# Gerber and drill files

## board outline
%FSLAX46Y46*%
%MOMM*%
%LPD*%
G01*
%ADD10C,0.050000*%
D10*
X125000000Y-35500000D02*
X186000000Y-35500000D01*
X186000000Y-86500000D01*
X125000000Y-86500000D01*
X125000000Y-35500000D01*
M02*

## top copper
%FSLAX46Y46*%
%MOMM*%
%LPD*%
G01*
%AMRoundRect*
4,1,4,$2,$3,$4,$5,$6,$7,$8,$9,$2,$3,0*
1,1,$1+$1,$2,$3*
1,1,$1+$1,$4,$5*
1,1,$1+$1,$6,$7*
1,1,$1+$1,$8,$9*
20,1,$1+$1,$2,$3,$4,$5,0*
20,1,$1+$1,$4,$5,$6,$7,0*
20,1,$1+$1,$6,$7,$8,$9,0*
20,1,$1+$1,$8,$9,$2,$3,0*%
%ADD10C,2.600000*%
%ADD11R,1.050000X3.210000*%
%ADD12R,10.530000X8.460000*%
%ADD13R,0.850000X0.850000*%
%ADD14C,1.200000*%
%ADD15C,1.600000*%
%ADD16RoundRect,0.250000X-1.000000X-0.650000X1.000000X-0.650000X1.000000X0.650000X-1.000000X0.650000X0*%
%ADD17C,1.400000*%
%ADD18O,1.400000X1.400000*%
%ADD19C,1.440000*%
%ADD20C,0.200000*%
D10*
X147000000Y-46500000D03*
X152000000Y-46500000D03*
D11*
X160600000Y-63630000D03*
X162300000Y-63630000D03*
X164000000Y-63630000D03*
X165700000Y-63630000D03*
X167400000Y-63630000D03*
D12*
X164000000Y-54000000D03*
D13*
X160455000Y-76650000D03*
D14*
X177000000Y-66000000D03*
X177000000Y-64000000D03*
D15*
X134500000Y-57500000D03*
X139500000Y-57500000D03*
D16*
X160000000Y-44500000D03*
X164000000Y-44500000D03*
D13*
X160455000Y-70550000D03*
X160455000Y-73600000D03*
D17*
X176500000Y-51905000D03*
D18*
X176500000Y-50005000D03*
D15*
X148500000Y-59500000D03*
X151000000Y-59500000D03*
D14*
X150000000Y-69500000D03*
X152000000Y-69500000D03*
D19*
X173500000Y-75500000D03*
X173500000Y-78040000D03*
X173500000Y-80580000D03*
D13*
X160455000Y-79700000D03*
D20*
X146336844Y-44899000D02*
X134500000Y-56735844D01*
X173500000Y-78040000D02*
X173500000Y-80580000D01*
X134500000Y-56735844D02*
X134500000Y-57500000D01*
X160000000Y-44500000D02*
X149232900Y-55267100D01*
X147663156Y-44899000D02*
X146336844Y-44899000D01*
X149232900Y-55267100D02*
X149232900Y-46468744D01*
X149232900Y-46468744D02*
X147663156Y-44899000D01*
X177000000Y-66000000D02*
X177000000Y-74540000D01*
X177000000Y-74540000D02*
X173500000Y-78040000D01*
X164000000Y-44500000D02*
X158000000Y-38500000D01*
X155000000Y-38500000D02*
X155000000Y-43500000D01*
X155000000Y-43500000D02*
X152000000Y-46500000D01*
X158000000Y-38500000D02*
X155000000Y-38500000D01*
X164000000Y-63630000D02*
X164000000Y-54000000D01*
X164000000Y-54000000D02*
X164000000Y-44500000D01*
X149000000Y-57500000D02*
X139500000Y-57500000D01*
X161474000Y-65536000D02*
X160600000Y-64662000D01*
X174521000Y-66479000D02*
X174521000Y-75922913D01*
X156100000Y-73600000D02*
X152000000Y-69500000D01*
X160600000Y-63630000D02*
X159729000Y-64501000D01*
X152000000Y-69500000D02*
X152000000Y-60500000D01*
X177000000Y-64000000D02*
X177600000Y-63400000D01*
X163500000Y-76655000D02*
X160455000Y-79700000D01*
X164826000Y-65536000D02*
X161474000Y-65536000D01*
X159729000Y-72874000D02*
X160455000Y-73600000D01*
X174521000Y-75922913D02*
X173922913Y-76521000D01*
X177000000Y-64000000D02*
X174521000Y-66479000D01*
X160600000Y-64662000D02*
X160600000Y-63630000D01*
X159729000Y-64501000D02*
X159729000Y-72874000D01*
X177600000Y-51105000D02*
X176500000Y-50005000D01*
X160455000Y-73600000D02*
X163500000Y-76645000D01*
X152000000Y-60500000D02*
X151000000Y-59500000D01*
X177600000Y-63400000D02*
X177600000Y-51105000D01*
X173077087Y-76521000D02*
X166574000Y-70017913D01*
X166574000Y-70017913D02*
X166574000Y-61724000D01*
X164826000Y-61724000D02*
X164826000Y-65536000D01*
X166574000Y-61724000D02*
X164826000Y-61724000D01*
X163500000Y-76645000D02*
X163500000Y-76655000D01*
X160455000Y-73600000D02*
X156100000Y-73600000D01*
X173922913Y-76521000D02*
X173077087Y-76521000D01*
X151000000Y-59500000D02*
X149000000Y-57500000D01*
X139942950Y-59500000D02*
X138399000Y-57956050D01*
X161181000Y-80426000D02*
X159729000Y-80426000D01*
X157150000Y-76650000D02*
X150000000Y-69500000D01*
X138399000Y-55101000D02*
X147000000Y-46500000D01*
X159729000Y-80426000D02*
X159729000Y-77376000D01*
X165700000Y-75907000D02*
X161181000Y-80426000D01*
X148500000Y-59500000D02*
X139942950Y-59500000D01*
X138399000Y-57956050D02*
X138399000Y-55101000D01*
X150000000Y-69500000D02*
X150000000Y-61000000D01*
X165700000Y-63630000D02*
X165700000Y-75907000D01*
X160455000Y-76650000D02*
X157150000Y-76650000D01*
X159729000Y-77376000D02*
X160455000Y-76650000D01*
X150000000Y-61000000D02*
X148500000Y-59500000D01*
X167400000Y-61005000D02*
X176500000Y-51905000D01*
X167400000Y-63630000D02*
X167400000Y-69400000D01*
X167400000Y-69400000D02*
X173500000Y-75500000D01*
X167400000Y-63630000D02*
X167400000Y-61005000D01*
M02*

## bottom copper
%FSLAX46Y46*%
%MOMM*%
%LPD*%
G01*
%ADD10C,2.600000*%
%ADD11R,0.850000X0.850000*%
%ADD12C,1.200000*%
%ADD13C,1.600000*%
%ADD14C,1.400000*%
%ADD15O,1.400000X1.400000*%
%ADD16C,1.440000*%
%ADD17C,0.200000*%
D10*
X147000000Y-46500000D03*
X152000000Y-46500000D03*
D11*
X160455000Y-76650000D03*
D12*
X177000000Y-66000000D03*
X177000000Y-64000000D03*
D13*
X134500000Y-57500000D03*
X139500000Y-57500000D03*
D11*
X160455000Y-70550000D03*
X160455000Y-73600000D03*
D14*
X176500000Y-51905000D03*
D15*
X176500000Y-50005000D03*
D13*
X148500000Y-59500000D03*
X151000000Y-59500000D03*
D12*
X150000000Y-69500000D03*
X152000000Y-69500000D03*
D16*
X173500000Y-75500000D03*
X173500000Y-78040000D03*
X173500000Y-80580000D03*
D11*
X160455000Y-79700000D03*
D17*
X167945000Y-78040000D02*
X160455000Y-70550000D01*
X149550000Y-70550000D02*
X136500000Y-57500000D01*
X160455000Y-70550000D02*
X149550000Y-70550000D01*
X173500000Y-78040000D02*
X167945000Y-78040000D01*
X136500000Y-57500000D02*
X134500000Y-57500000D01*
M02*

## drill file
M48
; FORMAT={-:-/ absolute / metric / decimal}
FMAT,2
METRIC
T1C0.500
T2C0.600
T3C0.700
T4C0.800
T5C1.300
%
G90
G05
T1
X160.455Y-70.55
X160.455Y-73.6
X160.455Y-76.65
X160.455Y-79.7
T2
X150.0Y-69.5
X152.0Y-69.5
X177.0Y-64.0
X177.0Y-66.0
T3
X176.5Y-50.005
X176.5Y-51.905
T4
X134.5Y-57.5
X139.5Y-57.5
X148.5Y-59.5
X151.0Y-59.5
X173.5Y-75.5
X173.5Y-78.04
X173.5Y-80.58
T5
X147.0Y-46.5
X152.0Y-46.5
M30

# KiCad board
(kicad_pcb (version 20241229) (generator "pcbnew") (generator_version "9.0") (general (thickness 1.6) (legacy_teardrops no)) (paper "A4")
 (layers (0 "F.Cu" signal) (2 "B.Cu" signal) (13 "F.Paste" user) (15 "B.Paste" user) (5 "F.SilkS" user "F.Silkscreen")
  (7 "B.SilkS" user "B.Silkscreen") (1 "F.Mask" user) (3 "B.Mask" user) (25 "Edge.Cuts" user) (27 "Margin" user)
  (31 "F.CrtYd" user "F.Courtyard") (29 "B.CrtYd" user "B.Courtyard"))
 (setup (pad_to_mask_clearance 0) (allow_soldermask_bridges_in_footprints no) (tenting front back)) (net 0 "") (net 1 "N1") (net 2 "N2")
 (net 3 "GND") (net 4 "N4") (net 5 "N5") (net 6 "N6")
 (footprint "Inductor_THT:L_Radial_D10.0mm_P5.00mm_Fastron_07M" (layer "F.Cu") (at 147 46.5)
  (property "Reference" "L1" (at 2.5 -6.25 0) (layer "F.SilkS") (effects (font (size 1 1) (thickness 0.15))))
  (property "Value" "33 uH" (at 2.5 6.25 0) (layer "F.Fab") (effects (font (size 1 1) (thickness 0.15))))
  (pad "1" thru_hole circle (at 0 0) (size 2.6 2.6) (drill 1.3) (layers "*.Cu" "*.Mask") (remove_unused_layers no) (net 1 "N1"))
  (pad "2" thru_hole circle (at 5 0) (size 2.6 2.6) (drill 1.3) (layers "*.Cu" "*.Mask") (remove_unused_layers no) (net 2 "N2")))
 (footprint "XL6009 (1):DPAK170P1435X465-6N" (layer "F.Cu") (at 164 57.5 90)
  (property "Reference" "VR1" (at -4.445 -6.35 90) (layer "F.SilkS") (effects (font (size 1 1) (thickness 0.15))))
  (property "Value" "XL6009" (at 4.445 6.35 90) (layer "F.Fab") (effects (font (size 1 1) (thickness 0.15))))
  (pad "1" smd rect (at -6.13 -3.4 90) (size 3.21 1.05) (layers "F.Cu" "F.Mask" "F.Paste") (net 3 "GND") (solder_mask_margin 0.102))
  (pad "2" smd rect (at -6.13 -1.7 90) (size 3.21 1.05) (layers "F.Cu" "F.Mask" "F.Paste") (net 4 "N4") (solder_mask_margin 0.102))
  (pad "3" smd rect (at -6.13 0 90) (size 3.21 1.05) (layers "F.Cu" "F.Mask" "F.Paste") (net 2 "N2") (solder_mask_margin 0.102))
  (pad "4" smd rect (at -6.13 1.7 90) (size 3.21 1.05) (layers "F.Cu" "F.Mask" "F.Paste") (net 1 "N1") (solder_mask_margin 0.102))
  (pad "5" smd rect (at -6.13 3.4 90) (size 3.21 1.05) (layers "F.Cu" "F.Mask" "F.Paste") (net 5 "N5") (solder_mask_margin 0.102))
  (pad "6" smd rect (at 3.5 0 90) (size 8.46 10.53) (layers "F.Cu" "F.Mask") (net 2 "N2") (solder_mask_margin 0.102)))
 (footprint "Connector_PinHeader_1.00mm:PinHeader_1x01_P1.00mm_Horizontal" (layer "F.Cu") (at 160.455 76.65)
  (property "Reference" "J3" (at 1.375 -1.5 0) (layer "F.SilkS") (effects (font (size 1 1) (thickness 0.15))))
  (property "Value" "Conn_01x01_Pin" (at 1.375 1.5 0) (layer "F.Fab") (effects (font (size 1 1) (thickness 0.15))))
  (pad "1" thru_hole rect (at 0 0) (size 0.85 0.85) (drill 0.5) (layers "*.Cu" "*.Mask") (remove_unused_layers no) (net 1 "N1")))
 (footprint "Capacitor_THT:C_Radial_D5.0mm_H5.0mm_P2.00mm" (layer "F.Cu") (at 177 66 90)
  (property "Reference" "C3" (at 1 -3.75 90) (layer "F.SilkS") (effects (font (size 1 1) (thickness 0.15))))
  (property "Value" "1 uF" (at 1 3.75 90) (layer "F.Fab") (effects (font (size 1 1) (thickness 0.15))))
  (pad "1" thru_hole circle (at 0 0 90) (size 1.2 1.2) (drill 0.6) (layers "*.Cu" "*.Mask") (remove_unused_layers no) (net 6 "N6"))
  (pad "2" thru_hole circle (at 2 0 90) (size 1.2 1.2) (drill 0.6) (layers "*.Cu" "*.Mask") (remove_unused_layers no) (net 3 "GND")))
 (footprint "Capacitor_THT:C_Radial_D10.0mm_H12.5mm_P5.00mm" (layer "F.Cu") (at 134.5 57.5)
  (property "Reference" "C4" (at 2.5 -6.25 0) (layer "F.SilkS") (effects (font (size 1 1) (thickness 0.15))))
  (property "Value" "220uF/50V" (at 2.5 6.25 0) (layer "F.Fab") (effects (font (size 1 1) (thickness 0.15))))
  (pad "1" thru_hole circle (at 0 0) (size 1.6 1.6) (drill 0.8) (layers "*.Cu" "*.Mask") (remove_unused_layers no) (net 6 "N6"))
  (pad "2" thru_hole circle (at 5 0) (size 1.6 1.6) (drill 0.8) (layers "*.Cu" "*.Mask") (remove_unused_layers no) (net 3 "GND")))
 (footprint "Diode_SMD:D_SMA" (layer "F.Cu") (at 162 44.5)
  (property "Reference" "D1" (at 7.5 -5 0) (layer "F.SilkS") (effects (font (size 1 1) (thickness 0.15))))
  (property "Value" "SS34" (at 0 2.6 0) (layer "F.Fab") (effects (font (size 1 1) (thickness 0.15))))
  (pad "1" smd roundrect (at -2 0) (size 2.5 1.8) (layers "F.Cu" "F.Mask" "F.Paste") (roundrect_rratio 0.1388888889) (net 6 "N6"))
  (pad "2" smd roundrect (at 2 0) (size 2.5 1.8) (layers "F.Cu" "F.Mask" "F.Paste") (roundrect_rratio 0.1388888889) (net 2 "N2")))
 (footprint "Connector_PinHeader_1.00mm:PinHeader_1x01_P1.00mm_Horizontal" (layer "F.Cu") (at 160.455 70.55)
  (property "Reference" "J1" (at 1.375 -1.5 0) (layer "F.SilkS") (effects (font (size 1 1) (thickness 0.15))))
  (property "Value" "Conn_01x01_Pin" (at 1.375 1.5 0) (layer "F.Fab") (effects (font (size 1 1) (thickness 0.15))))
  (pad "1" thru_hole rect (at 0 0) (size 0.85 0.85) (drill 0.5) (layers "*.Cu" "*.Mask") (remove_unused_layers no) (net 6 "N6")))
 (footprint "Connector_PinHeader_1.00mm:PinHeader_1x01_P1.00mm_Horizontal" (layer "F.Cu") (at 160.455 73.6)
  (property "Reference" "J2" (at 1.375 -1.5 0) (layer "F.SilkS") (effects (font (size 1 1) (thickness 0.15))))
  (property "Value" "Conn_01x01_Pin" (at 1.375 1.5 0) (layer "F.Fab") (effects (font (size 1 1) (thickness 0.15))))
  (pad "1" thru_hole rect (at 0 0) (size 0.85 0.85) (drill 0.5) (layers "*.Cu" "*.Mask") (remove_unused_layers no) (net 3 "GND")))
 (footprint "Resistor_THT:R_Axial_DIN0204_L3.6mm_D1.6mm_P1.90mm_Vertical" (layer "F.Cu") (at 176.5 51.905 90)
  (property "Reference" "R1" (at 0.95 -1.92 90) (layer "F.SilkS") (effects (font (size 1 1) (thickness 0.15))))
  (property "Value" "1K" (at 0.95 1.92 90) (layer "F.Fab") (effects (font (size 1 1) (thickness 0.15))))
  (pad "1" thru_hole circle (at 0 0 90) (size 1.4 1.4) (drill 0.7) (layers "*.Cu" "*.Mask") (remove_unused_layers no) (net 5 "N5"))
  (pad "2" thru_hole oval (at 1.9 0 90) (size 1.4 1.4) (drill 0.7) (layers "*.Cu" "*.Mask") (remove_unused_layers no) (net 3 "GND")))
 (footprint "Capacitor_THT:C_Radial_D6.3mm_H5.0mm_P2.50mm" (layer "F.Cu") (at 148.5 59.5)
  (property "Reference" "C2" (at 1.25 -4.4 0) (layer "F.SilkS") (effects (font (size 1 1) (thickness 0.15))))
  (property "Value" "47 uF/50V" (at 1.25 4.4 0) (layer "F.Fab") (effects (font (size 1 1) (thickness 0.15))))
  (pad "1" thru_hole circle (at 0 0) (size 1.6 1.6) (drill 0.8) (layers "*.Cu" "*.Mask") (remove_unused_layers no) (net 1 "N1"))
  (pad "2" thru_hole circle (at 2.5 0) (size 1.6 1.6) (drill 0.8) (layers "*.Cu" "*.Mask") (remove_unused_layers no) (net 3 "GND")))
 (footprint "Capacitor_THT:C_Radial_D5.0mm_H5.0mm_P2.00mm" (layer "F.Cu") (at 150 69.5)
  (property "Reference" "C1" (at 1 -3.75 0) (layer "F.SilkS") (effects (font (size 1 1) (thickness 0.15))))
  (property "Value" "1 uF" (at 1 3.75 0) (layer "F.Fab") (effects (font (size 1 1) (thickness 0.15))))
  (pad "1" thru_hole circle (at 0 0) (size 1.2 1.2) (drill 0.6) (layers "*.Cu" "*.Mask") (remove_unused_layers no) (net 1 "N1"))
  (pad "2" thru_hole circle (at 2 0) (size 1.2 1.2) (drill 0.6) (layers "*.Cu" "*.Mask") (remove_unused_layers no) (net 3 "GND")))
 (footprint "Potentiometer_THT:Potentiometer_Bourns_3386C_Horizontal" (layer "F.Cu") (at 173.5 75.5)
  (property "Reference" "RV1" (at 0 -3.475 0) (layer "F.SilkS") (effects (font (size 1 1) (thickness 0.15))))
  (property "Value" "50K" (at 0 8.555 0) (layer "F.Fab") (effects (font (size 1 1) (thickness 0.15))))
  (pad "1" thru_hole circle (at 0 0) (size 1.44 1.44) (drill 0.8) (layers "*.Cu" "*.Mask") (remove_unused_layers no) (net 5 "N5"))
  (pad "2" thru_hole circle (at 0 2.54) (size 1.44 1.44) (drill 0.8) (layers "*.Cu" "*.Mask") (remove_unused_layers no) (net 6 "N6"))
  (pad "3" thru_hole circle (at 0 5.08) (size 1.44 1.44) (drill 0.8) (layers "*.Cu" "*.Mask") (remove_unused_layers no) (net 6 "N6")))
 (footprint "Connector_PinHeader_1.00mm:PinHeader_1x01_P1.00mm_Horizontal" (layer "F.Cu") (at 160.455 79.7)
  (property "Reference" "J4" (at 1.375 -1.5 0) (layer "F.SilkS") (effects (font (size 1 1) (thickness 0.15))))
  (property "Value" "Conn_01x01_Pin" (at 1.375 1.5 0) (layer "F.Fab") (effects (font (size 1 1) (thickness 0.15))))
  (pad "1" thru_hole rect (at 0 0) (size 0.85 0.85) (drill 0.5) (layers "*.Cu" "*.Mask") (remove_unused_layers no) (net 3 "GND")))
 (gr_rect (start 125 35.5) (end 186 86.5) (stroke (width 0.05) (type default)) (fill no) (layer "Edge.Cuts"))
 (segment (start 146.336844 44.899) (end 134.5 56.735844) (width 0.2) (layer "F.Cu") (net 6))
 (segment (start 173.5 78.04) (end 173.5 80.58) (width 0.2) (layer "F.Cu") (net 6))
 (segment (start 134.5 56.735844) (end 134.5 57.5) (width 0.2) (layer "F.Cu") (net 6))
 (segment (start 160 44.5) (end 149.2329 55.2671) (width 0.2) (layer "F.Cu") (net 6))
 (segment (start 147.663156 44.899) (end 146.336844 44.899) (width 0.2) (layer "F.Cu") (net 6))
 (segment (start 149.2329 55.2671) (end 149.2329 46.468744) (width 0.2) (layer "F.Cu") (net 6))
 (segment (start 149.2329 46.468744) (end 147.663156 44.899) (width 0.2) (layer "F.Cu") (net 6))
 (segment (start 177 66) (end 177 74.54) (width 0.2) (layer "F.Cu") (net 6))
 (segment (start 177 74.54) (end 173.5 78.04) (width 0.2) (layer "F.Cu") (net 6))
 (segment (start 167.945 78.04) (end 160.455 70.55) (width 0.2) (layer "B.Cu") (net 6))
 (segment (start 149.55 70.55) (end 136.5 57.5) (width 0.2) (layer "B.Cu") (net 6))
 (segment (start 160.455 70.55) (end 149.55 70.55) (width 0.2) (layer "B.Cu") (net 6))
 (segment (start 173.5 78.04) (end 167.945 78.04) (width 0.2) (layer "B.Cu") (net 6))
 (segment (start 136.5 57.5) (end 134.5 57.5) (width 0.2) (layer "B.Cu") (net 6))
 (segment (start 164 44.5) (end 158 38.5) (width 0.2) (layer "F.Cu") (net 2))
 (segment (start 155 38.5) (end 155 43.5) (width 0.2) (layer "F.Cu") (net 2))
 (segment (start 155 43.5) (end 152 46.5) (width 0.2) (layer "F.Cu") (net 2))
 (segment (start 158 38.5) (end 155 38.5) (width 0.2) (layer "F.Cu") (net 2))
 (segment (start 164 63.63) (end 164 54) (width 0.2) (layer "F.Cu") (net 2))
 (segment (start 164 54) (end 164 44.5) (width 0.2) (layer "F.Cu") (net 2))
 (segment (start 149 57.5) (end 139.5 57.5) (width 0.2) (layer "F.Cu") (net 3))
 (segment (start 161.474 65.536) (end 160.6 64.662) (width 0.2) (layer "F.Cu") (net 3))
 (segment (start 174.521 66.479) (end 174.521 75.922913) (width 0.2) (layer "F.Cu") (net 3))
 (segment (start 156.1 73.6) (end 152 69.5) (width 0.2) (layer "F.Cu") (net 3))
 (segment (start 160.6 63.63) (end 159.729 64.501) (width 0.2) (layer "F.Cu") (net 3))
 (segment (start 152 69.5) (end 152 60.5) (width 0.2) (layer "F.Cu") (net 3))
 (segment (start 177 64) (end 177.6 63.4) (width 0.2) (layer "F.Cu") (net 3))
 (segment (start 163.5 76.655) (end 160.455 79.7) (width 0.2) (layer "F.Cu") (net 3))
 (segment (start 164.826 65.536) (end 161.474 65.536) (width 0.2) (layer "F.Cu") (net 3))
 (segment (start 159.729 72.874) (end 160.455 73.6) (width 0.2) (layer "F.Cu") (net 3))
 (segment (start 174.521 75.922913) (end 173.922913 76.521) (width 0.2) (layer "F.Cu") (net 3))
 (segment (start 177 64) (end 174.521 66.479) (width 0.2) (layer "F.Cu") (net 3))
 (segment (start 160.6 64.662) (end 160.6 63.63) (width 0.2) (layer "F.Cu") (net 3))
 (segment (start 159.729 64.501) (end 159.729 72.874) (width 0.2) (layer "F.Cu") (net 3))
 (segment (start 177.6 51.105) (end 176.5 50.005) (width 0.2) (layer "F.Cu") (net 3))
 (segment (start 160.455 73.6) (end 163.5 76.645) (width 0.2) (layer "F.Cu") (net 3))
 (segment (start 152 60.5) (end 151 59.5) (width 0.2) (layer "F.Cu") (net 3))
 (segment (start 177.6 63.4) (end 177.6 51.105) (width 0.2) (layer "F.Cu") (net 3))
 (segment (start 173.077087 76.521) (end 166.574 70.017913) (width 0.2) (layer "F.Cu") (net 3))
 (segment (start 166.574 70.017913) (end 166.574 61.724) (width 0.2) (layer "F.Cu") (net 3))
 (segment (start 164.826 61.724) (end 164.826 65.536) (width 0.2) (layer "F.Cu") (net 3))
 (segment (start 166.574 61.724) (end 164.826 61.724) (width 0.2) (layer "F.Cu") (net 3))
 (segment (start 163.5 76.645) (end 163.5 76.655) (width 0.2) (layer "F.Cu") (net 3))
 (segment (start 160.455 73.6) (end 156.1 73.6) (width 0.2) (layer "F.Cu") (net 3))
 (segment (start 173.922913 76.521) (end 173.077087 76.521) (width 0.2) (layer "F.Cu") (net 3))
 (segment (start 151 59.5) (end 149 57.5) (width 0.2) (layer "F.Cu") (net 3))
 (segment (start 139.94295 59.5) (end 138.399 57.95605) (width 0.2) (layer "F.Cu") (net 1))
 (segment (start 161.181 80.426) (end 159.729 80.426) (width 0.2) (layer "F.Cu") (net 1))
 (segment (start 157.15 76.65) (end 150 69.5) (width 0.2) (layer "F.Cu") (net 1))
 (segment (start 138.399 55.101) (end 147 46.5) (width 0.2) (layer "F.Cu") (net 1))
 (segment (start 159.729 80.426) (end 159.729 77.376) (width 0.2) (layer "F.Cu") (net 1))
 (segment (start 165.7 75.907) (end 161.181 80.426) (width 0.2) (layer "F.Cu") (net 1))
 (segment (start 148.5 59.5) (end 139.94295 59.5) (width 0.2) (layer "F.Cu") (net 1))
 (segment (start 138.399 57.95605) (end 138.399 55.101) (width 0.2) (layer "F.Cu") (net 1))
 (segment (start 150 69.5) (end 150 61) (width 0.2) (layer "F.Cu") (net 1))
 (segment (start 165.7 63.63) (end 165.7 75.907) (width 0.2) (layer "F.Cu") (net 1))
 (segment (start 160.455 76.65) (end 157.15 76.65) (width 0.2) (layer "F.Cu") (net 1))
 (segment (start 159.729 77.376) (end 160.455 76.65) (width 0.2) (layer "F.Cu") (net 1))
 (segment (start 150 61) (end 148.5 59.5) (width 0.2) (layer "F.Cu") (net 1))
 (segment (start 167.4 61.005) (end 176.5 51.905) (width 0.2) (layer "F.Cu") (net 5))
 (segment (start 167.4 63.63) (end 167.4 69.4) (width 0.2) (layer "F.Cu") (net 5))
 (segment (start 167.4 69.4) (end 173.5 75.5) (width 0.2) (layer "F.Cu") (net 5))
 (segment (start 167.4 63.63) (end 167.4 61.005) (width 0.2) (layer "F.Cu") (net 5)))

